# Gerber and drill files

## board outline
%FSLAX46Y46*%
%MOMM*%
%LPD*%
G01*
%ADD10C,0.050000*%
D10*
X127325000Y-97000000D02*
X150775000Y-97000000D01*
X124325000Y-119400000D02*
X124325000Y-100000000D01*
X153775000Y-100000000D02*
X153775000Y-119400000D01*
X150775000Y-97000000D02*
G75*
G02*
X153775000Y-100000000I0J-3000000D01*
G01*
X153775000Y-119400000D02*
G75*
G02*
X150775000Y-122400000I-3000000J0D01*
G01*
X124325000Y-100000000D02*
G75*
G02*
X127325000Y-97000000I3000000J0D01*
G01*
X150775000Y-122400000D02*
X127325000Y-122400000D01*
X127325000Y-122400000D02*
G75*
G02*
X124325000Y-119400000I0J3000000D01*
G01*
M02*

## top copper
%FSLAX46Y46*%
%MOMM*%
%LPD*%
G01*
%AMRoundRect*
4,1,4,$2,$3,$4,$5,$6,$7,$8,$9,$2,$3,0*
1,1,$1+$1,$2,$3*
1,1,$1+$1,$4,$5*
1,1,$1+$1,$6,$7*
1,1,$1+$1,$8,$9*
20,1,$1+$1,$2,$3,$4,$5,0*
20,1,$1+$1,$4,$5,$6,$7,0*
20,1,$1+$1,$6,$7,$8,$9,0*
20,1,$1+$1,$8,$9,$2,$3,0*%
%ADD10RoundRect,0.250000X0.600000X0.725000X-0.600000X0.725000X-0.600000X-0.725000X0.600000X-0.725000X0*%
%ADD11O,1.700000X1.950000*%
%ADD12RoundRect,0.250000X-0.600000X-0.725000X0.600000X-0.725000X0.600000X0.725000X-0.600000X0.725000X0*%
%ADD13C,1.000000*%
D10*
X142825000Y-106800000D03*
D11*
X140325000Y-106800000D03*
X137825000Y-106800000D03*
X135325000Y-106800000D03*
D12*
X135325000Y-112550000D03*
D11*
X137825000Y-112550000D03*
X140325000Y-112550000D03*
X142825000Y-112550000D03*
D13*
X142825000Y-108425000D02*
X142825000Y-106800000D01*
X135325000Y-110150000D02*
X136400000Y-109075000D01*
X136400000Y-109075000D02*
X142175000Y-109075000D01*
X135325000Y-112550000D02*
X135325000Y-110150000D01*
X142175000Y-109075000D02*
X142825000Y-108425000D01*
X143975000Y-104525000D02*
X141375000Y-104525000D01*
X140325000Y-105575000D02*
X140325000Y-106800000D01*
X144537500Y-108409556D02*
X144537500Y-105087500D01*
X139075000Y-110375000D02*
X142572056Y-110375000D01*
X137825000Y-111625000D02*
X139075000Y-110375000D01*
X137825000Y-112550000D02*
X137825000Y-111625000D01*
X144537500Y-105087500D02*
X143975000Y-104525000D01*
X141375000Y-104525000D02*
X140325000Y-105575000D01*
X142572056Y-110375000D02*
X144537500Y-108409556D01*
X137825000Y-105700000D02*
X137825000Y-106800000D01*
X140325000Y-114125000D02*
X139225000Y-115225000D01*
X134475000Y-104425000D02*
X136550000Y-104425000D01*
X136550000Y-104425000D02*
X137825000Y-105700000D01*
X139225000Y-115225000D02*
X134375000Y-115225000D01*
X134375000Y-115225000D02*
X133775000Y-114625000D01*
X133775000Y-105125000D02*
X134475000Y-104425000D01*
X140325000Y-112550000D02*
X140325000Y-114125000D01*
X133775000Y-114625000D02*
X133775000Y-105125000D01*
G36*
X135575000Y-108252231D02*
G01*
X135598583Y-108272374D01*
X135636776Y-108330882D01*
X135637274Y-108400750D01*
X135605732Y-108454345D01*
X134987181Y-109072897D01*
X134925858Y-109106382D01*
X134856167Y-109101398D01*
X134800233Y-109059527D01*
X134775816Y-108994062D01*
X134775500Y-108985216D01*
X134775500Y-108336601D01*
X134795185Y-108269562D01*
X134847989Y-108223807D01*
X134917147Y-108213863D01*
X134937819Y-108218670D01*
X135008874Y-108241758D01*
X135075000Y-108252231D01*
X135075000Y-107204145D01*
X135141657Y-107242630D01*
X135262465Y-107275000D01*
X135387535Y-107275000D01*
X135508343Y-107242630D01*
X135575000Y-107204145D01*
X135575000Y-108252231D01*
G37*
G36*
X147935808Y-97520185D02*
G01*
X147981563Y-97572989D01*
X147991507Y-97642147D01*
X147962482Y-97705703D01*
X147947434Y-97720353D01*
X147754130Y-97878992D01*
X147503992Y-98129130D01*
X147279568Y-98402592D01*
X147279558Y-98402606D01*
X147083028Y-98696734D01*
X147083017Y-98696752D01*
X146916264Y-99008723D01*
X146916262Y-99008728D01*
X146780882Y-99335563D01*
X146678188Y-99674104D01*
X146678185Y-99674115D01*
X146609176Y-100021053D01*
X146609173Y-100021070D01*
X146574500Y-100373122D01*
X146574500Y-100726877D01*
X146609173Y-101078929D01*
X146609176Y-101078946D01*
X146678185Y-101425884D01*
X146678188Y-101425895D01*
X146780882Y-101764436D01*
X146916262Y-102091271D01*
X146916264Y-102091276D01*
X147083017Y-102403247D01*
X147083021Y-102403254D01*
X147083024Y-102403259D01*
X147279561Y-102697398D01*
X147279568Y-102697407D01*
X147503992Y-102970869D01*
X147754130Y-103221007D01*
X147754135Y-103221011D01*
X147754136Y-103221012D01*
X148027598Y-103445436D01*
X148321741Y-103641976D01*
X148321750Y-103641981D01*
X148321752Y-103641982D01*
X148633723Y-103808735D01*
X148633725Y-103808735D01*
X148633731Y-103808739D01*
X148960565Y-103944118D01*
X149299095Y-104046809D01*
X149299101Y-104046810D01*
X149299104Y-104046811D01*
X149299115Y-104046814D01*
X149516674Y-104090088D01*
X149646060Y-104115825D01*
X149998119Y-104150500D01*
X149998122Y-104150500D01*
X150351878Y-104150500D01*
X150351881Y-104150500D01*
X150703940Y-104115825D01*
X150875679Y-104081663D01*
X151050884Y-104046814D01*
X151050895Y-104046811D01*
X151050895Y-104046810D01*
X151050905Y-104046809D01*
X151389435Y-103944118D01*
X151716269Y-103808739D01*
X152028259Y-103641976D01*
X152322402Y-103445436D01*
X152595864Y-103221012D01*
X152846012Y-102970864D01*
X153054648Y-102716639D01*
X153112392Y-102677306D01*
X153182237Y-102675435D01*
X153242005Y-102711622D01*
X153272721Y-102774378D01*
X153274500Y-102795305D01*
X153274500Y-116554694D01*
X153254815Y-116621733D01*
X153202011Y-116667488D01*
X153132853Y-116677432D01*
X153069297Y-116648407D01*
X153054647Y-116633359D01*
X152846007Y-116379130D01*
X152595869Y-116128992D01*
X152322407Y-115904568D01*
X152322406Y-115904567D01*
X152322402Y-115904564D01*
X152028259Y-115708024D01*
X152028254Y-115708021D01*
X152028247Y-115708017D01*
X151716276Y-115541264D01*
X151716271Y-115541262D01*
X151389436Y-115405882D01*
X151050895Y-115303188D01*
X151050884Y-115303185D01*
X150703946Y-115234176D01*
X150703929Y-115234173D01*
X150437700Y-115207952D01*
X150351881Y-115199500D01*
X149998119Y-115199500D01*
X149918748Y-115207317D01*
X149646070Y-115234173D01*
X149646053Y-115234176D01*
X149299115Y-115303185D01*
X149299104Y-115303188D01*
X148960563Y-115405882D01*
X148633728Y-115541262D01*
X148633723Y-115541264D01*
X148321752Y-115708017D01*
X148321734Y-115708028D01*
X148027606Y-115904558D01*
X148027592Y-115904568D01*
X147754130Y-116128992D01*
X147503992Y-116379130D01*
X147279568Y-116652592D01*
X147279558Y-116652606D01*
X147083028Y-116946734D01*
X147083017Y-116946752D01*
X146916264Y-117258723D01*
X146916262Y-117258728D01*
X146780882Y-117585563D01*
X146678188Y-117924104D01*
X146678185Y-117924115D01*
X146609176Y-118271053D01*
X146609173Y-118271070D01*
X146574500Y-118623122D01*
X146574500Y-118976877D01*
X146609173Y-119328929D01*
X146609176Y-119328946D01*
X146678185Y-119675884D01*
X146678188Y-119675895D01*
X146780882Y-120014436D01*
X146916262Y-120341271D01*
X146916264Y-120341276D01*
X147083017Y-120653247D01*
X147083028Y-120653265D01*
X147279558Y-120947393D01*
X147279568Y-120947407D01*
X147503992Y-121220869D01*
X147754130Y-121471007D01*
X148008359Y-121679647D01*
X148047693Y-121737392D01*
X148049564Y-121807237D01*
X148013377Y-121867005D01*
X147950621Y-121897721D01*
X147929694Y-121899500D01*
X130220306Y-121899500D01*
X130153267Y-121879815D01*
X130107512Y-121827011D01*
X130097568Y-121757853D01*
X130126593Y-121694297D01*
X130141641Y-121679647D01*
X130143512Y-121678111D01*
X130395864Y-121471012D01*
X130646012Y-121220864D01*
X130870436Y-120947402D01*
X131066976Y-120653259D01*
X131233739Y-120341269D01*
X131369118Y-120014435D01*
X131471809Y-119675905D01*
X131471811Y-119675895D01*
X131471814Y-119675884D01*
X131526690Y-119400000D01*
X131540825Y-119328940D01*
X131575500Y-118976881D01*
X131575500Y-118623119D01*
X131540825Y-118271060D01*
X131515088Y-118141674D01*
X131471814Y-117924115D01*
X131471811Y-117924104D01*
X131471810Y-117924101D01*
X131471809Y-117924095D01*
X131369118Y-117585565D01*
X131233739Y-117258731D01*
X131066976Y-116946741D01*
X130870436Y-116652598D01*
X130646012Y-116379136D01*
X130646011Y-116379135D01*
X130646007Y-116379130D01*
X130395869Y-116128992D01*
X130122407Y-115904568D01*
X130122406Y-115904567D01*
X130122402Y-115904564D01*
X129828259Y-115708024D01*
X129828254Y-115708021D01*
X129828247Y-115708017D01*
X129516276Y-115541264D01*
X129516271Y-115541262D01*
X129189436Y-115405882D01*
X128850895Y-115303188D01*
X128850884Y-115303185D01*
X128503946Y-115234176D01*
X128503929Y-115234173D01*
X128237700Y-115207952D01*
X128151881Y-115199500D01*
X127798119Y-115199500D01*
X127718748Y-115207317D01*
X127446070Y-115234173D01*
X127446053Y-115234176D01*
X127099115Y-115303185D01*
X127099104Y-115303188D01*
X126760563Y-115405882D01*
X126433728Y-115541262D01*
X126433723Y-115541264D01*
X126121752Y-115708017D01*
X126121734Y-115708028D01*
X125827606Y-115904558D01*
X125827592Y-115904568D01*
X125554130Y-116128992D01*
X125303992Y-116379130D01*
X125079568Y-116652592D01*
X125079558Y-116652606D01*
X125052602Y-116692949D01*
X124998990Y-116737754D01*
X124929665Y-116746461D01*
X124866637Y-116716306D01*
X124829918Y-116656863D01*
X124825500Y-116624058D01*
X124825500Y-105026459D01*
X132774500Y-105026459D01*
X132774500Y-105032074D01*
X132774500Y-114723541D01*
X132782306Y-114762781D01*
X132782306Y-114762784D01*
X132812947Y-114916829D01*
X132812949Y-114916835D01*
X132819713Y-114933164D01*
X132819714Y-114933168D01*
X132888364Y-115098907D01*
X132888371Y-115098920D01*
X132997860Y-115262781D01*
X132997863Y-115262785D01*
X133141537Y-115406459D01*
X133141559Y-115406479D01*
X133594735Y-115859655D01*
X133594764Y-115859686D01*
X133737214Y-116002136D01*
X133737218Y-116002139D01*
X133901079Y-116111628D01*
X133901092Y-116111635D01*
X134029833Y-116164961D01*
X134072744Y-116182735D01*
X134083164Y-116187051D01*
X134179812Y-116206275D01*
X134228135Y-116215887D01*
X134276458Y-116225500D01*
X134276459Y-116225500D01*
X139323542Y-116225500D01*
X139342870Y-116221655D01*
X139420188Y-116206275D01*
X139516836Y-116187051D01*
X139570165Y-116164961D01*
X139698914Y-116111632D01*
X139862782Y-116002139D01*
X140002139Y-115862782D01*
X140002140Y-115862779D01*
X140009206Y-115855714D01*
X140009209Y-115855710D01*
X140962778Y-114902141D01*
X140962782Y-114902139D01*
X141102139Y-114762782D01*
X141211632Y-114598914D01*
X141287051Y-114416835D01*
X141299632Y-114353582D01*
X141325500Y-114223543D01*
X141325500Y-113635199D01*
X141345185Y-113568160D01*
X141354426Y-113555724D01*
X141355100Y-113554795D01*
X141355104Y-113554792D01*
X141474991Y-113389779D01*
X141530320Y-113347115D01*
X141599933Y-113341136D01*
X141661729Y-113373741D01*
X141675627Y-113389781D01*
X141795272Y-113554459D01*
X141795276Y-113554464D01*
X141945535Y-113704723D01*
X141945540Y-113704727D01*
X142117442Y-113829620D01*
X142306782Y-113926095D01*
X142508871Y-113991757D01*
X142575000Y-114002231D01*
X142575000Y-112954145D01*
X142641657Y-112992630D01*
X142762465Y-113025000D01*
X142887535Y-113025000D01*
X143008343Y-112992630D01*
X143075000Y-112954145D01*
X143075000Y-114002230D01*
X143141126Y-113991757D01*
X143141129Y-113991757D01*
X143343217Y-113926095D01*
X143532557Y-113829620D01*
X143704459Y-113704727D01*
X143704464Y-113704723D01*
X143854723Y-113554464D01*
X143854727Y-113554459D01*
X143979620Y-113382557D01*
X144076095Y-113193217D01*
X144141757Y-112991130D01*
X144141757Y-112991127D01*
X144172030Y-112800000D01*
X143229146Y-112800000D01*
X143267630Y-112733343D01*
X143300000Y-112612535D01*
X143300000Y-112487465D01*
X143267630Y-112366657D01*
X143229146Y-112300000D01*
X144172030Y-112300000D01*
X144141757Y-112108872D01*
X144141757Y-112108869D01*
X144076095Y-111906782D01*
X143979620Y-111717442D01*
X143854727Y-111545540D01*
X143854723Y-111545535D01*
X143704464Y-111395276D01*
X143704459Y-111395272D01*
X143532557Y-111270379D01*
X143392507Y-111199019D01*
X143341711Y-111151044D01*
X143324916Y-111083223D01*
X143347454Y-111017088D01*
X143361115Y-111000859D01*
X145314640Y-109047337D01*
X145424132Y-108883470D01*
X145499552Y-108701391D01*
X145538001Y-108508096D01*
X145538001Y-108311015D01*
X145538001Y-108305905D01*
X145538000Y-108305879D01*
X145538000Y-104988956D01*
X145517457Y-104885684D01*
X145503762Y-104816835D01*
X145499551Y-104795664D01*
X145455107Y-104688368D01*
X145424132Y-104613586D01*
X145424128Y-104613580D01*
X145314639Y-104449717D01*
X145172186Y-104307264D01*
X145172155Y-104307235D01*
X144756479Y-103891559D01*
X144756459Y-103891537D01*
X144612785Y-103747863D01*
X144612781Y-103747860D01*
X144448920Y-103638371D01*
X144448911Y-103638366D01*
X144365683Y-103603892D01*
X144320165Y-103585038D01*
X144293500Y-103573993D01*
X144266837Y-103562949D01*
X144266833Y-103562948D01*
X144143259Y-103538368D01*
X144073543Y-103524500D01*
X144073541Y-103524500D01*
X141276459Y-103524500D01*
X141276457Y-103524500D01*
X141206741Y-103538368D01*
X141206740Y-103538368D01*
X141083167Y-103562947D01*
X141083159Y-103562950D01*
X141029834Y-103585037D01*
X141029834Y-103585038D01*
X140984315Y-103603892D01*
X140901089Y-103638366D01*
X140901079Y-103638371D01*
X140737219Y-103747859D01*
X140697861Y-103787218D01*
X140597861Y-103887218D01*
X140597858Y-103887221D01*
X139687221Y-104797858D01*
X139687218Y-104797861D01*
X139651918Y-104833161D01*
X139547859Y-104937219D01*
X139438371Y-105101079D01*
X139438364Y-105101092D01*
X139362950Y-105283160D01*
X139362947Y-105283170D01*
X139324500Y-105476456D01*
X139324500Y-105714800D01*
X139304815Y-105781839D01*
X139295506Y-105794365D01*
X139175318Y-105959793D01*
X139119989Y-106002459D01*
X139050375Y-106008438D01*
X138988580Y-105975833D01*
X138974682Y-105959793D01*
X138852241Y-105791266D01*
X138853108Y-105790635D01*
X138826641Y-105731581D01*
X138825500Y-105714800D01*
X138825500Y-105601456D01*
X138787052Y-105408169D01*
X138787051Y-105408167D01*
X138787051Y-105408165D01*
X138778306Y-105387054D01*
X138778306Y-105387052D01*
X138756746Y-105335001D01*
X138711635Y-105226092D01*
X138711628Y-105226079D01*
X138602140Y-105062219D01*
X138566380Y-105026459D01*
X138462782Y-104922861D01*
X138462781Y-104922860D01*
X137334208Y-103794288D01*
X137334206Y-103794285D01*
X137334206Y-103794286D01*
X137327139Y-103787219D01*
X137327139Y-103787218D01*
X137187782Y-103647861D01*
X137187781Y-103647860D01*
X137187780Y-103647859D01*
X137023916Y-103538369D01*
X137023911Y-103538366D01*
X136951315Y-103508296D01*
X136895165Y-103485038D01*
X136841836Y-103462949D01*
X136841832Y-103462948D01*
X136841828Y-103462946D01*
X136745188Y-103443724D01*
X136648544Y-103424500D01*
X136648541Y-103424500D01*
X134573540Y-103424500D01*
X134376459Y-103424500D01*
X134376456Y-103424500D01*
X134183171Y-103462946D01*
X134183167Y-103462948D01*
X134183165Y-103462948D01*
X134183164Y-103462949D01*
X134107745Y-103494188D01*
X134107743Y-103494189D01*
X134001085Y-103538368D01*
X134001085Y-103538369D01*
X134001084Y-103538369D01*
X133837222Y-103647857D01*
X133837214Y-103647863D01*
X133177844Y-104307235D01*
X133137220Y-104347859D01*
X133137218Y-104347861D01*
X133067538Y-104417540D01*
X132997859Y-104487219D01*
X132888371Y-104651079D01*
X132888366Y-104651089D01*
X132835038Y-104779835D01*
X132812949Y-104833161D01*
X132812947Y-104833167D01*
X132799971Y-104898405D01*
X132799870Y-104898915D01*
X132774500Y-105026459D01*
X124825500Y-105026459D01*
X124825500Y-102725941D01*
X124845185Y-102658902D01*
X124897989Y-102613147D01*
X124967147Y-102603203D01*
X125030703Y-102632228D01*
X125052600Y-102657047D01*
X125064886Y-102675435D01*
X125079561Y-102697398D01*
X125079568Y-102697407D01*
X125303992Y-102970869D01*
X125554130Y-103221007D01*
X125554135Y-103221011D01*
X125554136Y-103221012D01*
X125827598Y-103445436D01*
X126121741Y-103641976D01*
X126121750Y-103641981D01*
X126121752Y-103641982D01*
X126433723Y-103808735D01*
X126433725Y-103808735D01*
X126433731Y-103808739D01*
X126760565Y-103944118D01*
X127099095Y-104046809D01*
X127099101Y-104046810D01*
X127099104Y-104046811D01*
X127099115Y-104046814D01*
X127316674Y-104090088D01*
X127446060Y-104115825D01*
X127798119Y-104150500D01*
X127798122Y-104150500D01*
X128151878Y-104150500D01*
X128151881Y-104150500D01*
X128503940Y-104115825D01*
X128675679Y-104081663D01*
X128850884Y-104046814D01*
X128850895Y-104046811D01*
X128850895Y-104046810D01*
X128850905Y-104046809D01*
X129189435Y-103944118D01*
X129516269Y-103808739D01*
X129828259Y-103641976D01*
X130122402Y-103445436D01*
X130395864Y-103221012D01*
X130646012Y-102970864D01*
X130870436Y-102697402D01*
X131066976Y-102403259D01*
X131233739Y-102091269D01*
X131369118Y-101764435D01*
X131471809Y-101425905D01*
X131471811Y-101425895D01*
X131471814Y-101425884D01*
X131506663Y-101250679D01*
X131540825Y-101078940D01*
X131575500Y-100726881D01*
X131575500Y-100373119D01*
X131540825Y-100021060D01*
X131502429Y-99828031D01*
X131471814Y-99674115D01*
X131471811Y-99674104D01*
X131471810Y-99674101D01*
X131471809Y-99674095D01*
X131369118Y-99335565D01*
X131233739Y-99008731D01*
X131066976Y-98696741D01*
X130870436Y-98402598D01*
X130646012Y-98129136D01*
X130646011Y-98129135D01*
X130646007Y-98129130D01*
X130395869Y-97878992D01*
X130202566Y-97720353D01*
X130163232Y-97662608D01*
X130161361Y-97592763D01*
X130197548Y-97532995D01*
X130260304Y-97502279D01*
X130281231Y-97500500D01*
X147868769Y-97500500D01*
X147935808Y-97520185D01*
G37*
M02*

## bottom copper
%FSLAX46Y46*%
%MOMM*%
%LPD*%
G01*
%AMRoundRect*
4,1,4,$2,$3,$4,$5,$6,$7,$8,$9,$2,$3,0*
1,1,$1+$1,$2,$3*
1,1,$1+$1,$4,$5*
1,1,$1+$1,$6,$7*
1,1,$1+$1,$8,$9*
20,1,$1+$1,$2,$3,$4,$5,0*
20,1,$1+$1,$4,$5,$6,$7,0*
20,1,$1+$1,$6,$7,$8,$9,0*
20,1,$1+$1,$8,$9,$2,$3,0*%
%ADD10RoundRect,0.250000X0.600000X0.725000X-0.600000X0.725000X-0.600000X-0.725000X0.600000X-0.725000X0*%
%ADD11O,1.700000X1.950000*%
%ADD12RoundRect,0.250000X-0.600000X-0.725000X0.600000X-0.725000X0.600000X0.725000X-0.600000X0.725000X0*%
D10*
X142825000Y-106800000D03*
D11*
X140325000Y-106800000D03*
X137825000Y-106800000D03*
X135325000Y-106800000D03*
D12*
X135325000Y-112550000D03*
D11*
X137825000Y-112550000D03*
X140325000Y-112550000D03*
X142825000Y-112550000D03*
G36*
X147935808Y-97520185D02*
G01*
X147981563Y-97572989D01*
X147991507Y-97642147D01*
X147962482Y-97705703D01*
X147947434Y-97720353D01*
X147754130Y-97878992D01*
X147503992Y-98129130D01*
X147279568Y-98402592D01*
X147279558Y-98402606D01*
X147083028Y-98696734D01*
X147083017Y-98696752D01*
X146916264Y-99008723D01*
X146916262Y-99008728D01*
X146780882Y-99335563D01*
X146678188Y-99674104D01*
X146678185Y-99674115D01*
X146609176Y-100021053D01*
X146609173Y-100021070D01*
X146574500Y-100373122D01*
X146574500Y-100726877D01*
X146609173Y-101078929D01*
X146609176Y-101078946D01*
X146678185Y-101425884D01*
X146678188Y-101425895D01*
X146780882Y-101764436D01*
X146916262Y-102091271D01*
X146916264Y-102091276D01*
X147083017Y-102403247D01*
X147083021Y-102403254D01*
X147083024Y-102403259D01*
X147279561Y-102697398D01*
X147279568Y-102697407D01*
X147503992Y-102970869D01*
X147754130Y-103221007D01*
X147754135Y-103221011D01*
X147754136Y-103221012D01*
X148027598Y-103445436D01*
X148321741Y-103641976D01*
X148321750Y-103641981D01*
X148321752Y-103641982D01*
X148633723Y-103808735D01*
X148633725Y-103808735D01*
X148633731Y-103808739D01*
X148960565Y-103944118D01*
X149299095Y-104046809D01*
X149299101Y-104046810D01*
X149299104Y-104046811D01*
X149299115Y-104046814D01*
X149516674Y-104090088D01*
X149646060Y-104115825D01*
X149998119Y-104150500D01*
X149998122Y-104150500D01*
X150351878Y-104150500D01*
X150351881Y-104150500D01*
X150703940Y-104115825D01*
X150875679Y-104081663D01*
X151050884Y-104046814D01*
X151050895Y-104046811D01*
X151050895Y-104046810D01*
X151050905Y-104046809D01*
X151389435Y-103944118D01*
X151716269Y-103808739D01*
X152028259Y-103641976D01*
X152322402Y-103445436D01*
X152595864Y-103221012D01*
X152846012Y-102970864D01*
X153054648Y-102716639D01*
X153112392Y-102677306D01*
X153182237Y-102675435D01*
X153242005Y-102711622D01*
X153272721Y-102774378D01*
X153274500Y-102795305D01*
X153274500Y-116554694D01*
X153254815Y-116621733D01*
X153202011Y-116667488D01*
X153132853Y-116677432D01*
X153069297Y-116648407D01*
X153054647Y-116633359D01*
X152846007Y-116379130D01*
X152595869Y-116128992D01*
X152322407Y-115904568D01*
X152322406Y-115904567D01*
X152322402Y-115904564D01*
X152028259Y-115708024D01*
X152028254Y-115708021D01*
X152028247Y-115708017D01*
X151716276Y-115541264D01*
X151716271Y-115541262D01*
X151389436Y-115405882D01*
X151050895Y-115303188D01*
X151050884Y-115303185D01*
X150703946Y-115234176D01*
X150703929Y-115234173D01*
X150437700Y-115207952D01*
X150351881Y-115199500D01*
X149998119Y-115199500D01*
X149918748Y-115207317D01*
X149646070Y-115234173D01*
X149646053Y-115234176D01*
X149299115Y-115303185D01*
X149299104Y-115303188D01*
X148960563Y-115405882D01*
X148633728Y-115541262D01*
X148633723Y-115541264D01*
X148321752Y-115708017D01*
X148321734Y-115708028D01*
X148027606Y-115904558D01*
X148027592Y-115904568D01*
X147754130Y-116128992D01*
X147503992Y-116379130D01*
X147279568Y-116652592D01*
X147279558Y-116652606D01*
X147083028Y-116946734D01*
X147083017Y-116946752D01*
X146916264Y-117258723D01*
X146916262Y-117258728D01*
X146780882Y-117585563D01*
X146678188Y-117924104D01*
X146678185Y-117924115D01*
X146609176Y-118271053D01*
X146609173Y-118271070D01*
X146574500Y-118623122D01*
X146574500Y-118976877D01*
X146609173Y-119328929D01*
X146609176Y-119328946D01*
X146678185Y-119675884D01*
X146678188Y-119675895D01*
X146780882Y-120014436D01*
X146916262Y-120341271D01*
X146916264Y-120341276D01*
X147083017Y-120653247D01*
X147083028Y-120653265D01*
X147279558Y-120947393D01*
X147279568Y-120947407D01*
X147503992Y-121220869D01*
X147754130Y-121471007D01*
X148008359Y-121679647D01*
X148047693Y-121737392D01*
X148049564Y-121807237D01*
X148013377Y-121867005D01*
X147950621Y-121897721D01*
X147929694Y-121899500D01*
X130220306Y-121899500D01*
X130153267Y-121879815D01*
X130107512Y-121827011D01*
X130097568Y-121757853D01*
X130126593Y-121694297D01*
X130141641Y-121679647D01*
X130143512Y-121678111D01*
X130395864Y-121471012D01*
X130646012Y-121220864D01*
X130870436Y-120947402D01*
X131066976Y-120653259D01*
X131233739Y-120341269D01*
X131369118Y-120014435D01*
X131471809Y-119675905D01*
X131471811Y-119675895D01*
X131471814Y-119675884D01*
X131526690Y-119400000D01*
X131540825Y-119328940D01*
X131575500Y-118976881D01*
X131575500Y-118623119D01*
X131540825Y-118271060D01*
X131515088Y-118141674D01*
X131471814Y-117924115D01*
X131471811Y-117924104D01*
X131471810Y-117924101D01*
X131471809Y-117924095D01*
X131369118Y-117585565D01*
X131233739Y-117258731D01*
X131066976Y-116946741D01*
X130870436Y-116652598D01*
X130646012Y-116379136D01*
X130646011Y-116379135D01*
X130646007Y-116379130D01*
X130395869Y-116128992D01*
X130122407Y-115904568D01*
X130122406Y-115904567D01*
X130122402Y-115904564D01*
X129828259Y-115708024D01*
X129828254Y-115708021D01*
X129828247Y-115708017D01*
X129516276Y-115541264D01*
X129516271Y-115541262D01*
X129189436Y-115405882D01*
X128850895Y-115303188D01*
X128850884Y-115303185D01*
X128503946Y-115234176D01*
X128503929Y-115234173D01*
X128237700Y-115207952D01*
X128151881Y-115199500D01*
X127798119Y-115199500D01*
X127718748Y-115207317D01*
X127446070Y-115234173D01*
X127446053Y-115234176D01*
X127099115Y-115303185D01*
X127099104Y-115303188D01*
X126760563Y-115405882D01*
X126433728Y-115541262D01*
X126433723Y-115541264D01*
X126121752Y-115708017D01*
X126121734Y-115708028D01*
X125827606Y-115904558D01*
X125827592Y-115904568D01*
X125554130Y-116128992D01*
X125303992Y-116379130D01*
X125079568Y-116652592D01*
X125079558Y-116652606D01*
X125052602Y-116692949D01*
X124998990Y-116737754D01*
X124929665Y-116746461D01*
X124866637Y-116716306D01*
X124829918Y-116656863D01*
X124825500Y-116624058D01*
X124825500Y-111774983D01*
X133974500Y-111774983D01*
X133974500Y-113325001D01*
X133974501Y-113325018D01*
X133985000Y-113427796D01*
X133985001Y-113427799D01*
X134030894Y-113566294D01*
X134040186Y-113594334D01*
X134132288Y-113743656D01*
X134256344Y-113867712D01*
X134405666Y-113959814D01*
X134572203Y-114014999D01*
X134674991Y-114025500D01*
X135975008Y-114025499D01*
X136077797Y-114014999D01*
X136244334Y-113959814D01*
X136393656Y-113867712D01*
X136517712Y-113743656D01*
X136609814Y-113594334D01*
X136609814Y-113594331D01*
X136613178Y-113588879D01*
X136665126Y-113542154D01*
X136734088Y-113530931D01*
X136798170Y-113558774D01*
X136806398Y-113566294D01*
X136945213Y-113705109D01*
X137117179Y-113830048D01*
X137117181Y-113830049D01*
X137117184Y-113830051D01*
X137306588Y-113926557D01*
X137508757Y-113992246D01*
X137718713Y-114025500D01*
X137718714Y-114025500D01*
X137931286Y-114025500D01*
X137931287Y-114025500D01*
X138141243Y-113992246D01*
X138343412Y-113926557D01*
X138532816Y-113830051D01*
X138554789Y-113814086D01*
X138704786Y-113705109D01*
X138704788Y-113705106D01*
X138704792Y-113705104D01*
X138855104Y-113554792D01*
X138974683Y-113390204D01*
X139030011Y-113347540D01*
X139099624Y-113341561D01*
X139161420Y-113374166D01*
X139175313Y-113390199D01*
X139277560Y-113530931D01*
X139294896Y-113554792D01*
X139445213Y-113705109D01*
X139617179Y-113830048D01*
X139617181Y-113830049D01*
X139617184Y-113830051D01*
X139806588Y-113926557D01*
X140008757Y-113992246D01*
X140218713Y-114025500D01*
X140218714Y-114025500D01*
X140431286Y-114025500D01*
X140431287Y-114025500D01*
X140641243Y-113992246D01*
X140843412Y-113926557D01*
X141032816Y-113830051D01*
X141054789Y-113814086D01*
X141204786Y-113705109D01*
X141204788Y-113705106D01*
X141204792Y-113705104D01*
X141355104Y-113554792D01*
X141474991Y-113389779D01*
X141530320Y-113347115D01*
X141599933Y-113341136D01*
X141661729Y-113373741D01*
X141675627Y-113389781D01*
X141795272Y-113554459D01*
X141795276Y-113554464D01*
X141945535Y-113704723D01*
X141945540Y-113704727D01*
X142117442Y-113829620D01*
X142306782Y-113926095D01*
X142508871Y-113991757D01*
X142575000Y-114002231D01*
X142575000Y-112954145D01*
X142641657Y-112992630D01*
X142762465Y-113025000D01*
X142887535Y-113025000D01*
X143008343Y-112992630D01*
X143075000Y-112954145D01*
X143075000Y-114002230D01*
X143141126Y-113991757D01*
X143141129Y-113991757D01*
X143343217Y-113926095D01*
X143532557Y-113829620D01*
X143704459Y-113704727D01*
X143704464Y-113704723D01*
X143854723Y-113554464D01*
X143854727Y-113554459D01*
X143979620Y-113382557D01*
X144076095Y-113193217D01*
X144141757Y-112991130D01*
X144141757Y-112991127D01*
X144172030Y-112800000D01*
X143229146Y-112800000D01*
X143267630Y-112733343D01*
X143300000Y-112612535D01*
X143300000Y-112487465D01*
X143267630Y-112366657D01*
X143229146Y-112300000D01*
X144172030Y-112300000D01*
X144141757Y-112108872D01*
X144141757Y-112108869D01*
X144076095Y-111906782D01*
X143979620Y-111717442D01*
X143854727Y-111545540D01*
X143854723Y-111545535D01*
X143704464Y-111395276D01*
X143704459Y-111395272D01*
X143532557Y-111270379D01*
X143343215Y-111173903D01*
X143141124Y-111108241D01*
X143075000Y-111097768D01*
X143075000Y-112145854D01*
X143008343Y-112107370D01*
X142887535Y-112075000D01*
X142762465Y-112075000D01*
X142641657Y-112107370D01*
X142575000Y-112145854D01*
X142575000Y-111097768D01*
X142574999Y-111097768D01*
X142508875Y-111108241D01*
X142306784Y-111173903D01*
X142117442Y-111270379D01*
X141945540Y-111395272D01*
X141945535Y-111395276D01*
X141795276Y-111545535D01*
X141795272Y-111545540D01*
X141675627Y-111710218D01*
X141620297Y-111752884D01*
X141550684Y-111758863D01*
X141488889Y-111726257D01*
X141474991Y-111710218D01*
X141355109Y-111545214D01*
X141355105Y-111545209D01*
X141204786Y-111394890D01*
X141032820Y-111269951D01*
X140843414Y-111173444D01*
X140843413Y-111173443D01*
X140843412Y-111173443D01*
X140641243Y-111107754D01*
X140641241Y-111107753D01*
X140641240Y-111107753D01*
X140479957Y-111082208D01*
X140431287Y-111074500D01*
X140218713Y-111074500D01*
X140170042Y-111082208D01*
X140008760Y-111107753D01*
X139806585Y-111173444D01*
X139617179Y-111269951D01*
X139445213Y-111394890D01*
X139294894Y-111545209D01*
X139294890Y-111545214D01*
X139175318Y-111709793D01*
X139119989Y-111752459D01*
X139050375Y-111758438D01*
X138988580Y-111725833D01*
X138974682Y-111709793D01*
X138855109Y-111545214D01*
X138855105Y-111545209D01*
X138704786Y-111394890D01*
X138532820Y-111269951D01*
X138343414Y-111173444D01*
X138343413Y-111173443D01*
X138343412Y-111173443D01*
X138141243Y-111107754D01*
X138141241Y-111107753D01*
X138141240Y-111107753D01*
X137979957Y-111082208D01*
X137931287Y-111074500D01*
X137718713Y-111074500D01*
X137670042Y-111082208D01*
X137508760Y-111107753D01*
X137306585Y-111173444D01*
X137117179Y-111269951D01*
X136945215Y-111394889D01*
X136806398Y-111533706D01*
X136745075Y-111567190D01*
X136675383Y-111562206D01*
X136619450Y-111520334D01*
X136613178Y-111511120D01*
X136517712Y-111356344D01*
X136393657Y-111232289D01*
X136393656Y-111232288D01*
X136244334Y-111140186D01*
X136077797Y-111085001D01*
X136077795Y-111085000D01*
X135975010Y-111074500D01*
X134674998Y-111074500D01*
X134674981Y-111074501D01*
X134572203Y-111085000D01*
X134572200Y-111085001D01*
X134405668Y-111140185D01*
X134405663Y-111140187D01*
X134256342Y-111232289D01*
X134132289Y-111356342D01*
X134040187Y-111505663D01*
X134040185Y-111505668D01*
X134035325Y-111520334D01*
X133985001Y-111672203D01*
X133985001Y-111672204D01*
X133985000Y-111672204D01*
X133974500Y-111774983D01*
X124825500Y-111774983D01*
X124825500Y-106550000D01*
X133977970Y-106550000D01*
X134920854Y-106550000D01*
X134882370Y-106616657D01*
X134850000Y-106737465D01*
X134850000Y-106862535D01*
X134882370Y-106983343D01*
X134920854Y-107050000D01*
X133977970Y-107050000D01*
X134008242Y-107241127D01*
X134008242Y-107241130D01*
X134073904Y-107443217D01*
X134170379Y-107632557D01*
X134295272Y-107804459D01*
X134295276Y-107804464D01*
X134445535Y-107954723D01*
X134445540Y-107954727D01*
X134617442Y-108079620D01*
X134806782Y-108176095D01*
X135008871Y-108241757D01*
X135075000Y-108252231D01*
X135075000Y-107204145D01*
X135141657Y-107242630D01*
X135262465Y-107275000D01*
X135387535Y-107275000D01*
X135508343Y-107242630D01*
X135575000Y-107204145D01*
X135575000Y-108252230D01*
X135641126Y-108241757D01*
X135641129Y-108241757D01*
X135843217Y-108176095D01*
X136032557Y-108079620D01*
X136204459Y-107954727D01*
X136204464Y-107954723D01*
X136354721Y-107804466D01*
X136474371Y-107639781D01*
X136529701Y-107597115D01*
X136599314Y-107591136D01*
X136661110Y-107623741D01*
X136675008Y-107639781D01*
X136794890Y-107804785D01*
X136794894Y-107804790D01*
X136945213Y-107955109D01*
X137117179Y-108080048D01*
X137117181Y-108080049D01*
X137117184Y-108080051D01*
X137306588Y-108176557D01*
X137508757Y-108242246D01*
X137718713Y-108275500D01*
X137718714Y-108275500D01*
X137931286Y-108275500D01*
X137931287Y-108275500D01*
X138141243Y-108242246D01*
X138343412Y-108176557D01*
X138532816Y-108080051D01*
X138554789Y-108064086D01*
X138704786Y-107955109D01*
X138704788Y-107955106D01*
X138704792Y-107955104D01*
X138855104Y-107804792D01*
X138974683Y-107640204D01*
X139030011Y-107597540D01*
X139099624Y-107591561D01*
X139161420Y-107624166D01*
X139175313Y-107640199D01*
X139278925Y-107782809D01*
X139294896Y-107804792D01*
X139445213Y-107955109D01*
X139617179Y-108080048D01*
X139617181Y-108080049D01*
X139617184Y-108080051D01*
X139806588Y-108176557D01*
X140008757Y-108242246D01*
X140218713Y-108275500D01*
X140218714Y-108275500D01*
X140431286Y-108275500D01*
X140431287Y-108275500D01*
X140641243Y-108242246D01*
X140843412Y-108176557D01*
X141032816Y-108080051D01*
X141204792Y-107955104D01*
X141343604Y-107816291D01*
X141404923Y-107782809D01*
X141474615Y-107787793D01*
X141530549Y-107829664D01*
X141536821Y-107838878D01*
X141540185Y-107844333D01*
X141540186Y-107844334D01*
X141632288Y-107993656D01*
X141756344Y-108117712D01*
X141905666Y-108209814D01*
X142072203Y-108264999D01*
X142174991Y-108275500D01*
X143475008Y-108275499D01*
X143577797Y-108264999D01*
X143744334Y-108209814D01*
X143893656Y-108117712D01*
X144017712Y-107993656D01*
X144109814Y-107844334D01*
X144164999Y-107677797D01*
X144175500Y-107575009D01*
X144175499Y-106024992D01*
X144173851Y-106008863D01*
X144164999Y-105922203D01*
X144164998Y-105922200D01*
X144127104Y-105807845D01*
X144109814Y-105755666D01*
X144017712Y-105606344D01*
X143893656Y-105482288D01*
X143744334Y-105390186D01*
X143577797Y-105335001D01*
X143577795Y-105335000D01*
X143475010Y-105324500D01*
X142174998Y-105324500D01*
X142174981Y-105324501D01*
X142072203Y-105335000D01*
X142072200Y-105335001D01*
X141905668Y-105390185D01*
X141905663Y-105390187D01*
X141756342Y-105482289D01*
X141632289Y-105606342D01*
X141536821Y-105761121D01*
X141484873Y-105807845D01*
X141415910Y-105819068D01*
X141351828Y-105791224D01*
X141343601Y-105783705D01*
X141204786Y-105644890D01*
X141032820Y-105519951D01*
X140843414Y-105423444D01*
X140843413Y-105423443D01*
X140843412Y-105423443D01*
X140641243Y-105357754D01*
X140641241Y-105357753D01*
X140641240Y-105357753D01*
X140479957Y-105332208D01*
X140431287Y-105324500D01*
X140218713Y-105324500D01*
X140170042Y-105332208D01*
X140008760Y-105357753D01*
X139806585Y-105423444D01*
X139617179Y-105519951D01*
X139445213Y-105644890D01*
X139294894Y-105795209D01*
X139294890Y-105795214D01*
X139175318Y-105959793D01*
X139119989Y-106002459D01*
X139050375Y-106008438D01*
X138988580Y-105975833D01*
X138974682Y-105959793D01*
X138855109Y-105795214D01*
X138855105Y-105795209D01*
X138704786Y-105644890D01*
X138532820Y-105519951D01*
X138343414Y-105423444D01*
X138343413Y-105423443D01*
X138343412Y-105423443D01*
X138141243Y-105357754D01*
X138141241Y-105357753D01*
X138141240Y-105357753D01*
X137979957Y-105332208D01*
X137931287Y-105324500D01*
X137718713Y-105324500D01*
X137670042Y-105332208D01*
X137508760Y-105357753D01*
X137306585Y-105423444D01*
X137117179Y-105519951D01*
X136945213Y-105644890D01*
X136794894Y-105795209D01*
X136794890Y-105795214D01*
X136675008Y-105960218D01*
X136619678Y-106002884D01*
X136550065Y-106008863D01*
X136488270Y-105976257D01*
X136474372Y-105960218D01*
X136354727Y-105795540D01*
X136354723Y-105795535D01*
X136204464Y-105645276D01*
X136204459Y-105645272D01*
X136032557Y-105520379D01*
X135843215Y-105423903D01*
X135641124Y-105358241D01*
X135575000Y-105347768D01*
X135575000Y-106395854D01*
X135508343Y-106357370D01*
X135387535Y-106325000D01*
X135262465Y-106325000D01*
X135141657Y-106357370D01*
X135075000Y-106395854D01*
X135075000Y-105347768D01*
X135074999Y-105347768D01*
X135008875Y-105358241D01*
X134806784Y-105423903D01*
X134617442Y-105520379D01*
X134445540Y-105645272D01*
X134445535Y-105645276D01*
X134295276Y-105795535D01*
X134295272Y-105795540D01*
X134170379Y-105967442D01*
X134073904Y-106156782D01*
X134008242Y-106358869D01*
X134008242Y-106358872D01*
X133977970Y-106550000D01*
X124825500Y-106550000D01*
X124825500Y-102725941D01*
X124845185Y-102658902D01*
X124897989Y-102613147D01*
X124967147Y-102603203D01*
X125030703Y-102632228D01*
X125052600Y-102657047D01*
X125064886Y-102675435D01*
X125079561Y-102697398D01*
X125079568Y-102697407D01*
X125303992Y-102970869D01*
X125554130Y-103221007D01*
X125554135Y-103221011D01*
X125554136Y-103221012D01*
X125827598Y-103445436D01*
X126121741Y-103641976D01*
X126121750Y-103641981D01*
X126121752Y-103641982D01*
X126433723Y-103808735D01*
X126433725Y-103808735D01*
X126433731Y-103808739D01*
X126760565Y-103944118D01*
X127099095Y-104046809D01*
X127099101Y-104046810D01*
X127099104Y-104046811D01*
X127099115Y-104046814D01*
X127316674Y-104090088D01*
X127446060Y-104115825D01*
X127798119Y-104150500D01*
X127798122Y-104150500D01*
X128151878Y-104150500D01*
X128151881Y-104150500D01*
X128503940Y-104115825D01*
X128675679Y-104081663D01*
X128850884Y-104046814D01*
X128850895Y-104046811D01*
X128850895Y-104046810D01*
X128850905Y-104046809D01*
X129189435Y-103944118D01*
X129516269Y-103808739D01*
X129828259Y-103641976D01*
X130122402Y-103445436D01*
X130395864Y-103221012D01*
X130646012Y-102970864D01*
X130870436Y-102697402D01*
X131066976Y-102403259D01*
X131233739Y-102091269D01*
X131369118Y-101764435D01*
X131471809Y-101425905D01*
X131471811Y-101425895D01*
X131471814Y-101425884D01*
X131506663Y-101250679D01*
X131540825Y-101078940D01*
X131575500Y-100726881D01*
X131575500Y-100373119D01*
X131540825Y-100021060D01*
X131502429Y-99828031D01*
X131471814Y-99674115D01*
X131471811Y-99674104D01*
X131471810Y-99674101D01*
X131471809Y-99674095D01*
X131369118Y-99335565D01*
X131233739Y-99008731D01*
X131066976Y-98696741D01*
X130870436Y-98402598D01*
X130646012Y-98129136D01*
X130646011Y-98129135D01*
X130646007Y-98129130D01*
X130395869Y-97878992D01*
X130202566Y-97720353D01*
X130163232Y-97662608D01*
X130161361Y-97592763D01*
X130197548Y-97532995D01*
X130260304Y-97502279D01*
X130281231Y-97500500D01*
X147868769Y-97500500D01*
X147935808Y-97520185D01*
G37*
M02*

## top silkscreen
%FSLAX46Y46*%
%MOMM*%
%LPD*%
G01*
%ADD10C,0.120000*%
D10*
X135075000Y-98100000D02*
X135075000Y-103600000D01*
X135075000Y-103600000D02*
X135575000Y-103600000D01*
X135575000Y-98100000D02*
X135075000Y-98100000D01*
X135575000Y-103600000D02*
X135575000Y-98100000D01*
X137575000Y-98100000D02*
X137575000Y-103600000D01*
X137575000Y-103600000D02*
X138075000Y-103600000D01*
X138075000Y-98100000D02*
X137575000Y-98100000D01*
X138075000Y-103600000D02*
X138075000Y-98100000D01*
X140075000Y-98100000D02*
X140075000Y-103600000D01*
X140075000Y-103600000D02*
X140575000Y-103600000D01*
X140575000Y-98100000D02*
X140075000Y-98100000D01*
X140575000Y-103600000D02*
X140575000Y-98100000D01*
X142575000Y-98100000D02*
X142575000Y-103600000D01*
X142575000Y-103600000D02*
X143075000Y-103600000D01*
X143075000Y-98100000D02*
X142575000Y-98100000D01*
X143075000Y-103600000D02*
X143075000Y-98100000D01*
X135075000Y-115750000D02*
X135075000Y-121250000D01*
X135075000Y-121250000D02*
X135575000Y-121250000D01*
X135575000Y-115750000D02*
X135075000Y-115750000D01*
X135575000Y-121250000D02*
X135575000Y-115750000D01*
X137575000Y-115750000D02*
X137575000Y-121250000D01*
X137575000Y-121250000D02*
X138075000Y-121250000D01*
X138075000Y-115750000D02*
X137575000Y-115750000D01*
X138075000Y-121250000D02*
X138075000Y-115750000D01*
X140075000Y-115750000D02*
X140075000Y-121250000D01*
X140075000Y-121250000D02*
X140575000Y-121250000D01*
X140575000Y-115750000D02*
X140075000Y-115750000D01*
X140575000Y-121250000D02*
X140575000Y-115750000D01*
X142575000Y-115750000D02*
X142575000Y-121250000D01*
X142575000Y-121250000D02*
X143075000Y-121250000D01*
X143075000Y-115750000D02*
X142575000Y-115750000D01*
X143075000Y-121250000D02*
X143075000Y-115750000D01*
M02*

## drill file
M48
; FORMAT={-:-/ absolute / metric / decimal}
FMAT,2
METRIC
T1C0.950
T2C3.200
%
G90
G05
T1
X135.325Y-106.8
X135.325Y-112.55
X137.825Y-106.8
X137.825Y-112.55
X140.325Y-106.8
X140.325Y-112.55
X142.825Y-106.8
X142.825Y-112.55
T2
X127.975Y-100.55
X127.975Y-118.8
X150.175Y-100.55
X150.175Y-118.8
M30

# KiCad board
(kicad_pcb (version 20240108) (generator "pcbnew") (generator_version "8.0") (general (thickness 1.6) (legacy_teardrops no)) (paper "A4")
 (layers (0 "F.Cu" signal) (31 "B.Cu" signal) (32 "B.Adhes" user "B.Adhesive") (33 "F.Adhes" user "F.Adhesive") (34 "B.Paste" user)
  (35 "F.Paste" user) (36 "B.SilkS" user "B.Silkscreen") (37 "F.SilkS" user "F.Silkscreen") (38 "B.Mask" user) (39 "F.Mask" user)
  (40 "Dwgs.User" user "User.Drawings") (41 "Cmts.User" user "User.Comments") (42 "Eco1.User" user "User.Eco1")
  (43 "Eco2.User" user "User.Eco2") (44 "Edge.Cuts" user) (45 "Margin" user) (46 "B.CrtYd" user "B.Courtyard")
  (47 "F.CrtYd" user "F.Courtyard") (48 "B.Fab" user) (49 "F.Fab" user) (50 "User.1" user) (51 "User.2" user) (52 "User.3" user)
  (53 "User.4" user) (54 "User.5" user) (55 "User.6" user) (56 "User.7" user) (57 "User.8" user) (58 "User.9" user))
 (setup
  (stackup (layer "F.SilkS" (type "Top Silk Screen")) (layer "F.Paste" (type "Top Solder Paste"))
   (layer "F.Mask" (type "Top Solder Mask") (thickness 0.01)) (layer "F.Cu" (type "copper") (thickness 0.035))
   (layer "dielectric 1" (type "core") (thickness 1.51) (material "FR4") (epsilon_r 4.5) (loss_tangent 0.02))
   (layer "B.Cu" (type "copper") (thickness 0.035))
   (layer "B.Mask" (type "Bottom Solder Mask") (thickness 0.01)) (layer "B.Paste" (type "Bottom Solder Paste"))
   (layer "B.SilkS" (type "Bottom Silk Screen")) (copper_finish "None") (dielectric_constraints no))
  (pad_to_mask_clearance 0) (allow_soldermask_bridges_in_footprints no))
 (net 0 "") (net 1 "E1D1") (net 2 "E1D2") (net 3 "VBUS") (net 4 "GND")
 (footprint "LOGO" (layer "F.Cu") (at 146.350293 109.852368)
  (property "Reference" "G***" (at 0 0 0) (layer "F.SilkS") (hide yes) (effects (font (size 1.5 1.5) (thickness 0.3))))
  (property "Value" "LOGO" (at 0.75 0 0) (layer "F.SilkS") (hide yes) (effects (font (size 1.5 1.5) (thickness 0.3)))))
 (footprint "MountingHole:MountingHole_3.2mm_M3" (layer "F.Cu") (at 150.175 118.8)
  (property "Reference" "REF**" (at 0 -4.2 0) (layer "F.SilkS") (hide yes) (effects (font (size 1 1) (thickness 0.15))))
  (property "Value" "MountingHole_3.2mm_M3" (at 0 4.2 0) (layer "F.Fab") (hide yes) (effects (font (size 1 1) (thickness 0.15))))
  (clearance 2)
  (pad "" np_thru_hole circle (at 0 0) (size 3.2 3.2) (drill 3.2) (layers "*.Cu" "*.Mask")))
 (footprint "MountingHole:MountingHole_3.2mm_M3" (layer "F.Cu") (at 150.175 100.55)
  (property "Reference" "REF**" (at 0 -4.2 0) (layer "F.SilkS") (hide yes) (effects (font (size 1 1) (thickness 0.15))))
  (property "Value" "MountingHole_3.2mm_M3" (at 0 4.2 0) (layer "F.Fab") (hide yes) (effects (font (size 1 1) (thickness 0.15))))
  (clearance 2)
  (pad "" np_thru_hole circle (at 0 0) (size 3.2 3.2) (drill 3.2) (layers "*.Cu" "*.Mask")))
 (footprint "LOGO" (layer "F.Cu") (at 132.30565 109.62003)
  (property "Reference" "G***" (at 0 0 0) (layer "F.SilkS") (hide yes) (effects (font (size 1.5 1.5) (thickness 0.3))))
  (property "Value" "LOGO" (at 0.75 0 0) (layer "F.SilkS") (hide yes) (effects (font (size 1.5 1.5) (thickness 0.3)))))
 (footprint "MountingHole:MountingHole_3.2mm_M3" (layer "F.Cu") (at 127.975 118.8)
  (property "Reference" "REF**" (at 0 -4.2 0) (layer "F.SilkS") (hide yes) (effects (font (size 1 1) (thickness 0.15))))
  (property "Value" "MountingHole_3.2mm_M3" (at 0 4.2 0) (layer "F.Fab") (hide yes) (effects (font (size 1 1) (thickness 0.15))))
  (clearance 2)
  (pad "" np_thru_hole circle (at 0 0) (size 3.2 3.2) (drill 3.2) (layers "*.Cu" "*.Mask")))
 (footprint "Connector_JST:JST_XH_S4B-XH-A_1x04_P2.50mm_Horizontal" (layer "F.Cu") (at 142.825 106.8 180)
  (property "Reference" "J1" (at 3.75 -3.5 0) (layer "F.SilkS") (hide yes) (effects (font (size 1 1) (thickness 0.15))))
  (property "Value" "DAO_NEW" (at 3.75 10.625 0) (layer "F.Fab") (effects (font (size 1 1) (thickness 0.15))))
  (fp_line (start 7.75 8.7) (end 7.75 3.2) (stroke (width 0.12) (type solid)) (layer "F.SilkS"))
  (fp_line (start 7.75 3.2) (end 7.25 3.2) (stroke (width 0.12) (type solid)) (layer "F.SilkS"))
  (fp_line (start 7.25 8.7) (end 7.75 8.7) (stroke (width 0.12) (type solid)) (layer "F.SilkS"))
  (fp_line (start 7.25 3.2) (end 7.25 8.7) (stroke (width 0.12) (type solid)) (layer "F.SilkS"))
  (fp_line (start 5.25 8.7) (end 5.25 3.2) (stroke (width 0.12) (type solid)) (layer "F.SilkS"))
  (fp_line (start 5.25 3.2) (end 4.75 3.2) (stroke (width 0.12) (type solid)) (layer "F.SilkS"))
  (fp_line (start 4.75 8.7) (end 5.25 8.7) (stroke (width 0.12) (type solid)) (layer "F.SilkS"))
  (fp_line (start 4.75 3.2) (end 4.75 8.7) (stroke (width 0.12) (type solid)) (layer "F.SilkS"))
  (fp_line (start 2.75 8.7) (end 2.75 3.2) (stroke (width 0.12) (type solid)) (layer "F.SilkS"))
  (fp_line (start 2.75 3.2) (end 2.25 3.2) (stroke (width 0.12) (type solid)) (layer "F.SilkS"))
  (fp_line (start 2.25 8.7) (end 2.75 8.7) (stroke (width 0.12) (type solid)) (layer "F.SilkS"))
  (fp_line (start 2.25 3.2) (end 2.25 8.7) (stroke (width 0.12) (type solid)) (layer "F.SilkS"))
  (fp_line (start 0.25 8.7) (end 0.25 3.2) (stroke (width 0.12) (type solid)) (layer "F.SilkS"))
  (fp_line (start 0.25 3.2) (end -0.25 3.2) (stroke (width 0.12) (type solid)) (layer "F.SilkS"))
  (fp_line (start -0.25 8.7) (end 0.25 8.7) (stroke (width 0.12) (type solid)) (layer "F.SilkS"))
  (fp_line (start -0.25 3.2) (end -0.25 8.7) (stroke (width 0.12) (type solid)) (layer "F.SilkS"))
  (pad "1" thru_hole roundrect (at 0 0 180) (size 1.7 1.95) (drill 0.95) (layers "*.Cu" "*.Mask") (remove_unused_layers no)
   (roundrect_rratio 0.147059) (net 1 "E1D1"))
  (pad "2" thru_hole oval (at 2.5 0 180) (size 1.7 1.95) (drill 0.95) (layers "*.Cu" "*.Mask") (remove_unused_layers no) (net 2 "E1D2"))
  (pad "3" thru_hole oval (at 5 0 180) (size 1.7 1.95) (drill 0.95) (layers "*.Cu" "*.Mask") (remove_unused_layers no) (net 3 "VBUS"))
  (pad "4" thru_hole oval (at 7.5 0 180) (size 1.7 1.95) (drill 0.95) (layers "*.Cu" "*.Mask") (remove_unused_layers no) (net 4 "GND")))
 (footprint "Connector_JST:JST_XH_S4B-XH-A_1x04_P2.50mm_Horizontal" (layer "F.Cu") (at 135.325 112.55)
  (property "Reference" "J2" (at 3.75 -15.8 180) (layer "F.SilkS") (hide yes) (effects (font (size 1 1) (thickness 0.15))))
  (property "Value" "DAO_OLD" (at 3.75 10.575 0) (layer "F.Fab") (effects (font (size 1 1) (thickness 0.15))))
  (fp_line (start -0.25 3.2) (end -0.25 8.7) (stroke (width 0.12) (type solid)) (layer "F.SilkS"))
  (fp_line (start -0.25 8.7) (end 0.25 8.7) (stroke (width 0.12) (type solid)) (layer "F.SilkS"))
  (fp_line (start 0.25 3.2) (end -0.25 3.2) (stroke (width 0.12) (type solid)) (layer "F.SilkS"))
  (fp_line (start 0.25 8.7) (end 0.25 3.2) (stroke (width 0.12) (type solid)) (layer "F.SilkS"))
  (fp_line (start 2.25 3.2) (end 2.25 8.7) (stroke (width 0.12) (type solid)) (layer "F.SilkS"))
  (fp_line (start 2.25 8.7) (end 2.75 8.7) (stroke (width 0.12) (type solid)) (layer "F.SilkS"))
  (fp_line (start 2.75 3.2) (end 2.25 3.2) (stroke (width 0.12) (type solid)) (layer "F.SilkS"))
  (fp_line (start 2.75 8.7) (end 2.75 3.2) (stroke (width 0.12) (type solid)) (layer "F.SilkS"))
  (fp_line (start 4.75 3.2) (end 4.75 8.7) (stroke (width 0.12) (type solid)) (layer "F.SilkS"))
  (fp_line (start 4.75 8.7) (end 5.25 8.7) (stroke (width 0.12) (type solid)) (layer "F.SilkS"))
  (fp_line (start 5.25 3.2) (end 4.75 3.2) (stroke (width 0.12) (type solid)) (layer "F.SilkS"))
  (fp_line (start 5.25 8.7) (end 5.25 3.2) (stroke (width 0.12) (type solid)) (layer "F.SilkS"))
  (fp_line (start 7.25 3.2) (end 7.25 8.7) (stroke (width 0.12) (type solid)) (layer "F.SilkS"))
  (fp_line (start 7.25 8.7) (end 7.75 8.7) (stroke (width 0.12) (type solid)) (layer "F.SilkS"))
  (fp_line (start 7.75 3.2) (end 7.25 3.2) (stroke (width 0.12) (type solid)) (layer "F.SilkS"))
  (fp_line (start 7.75 8.7) (end 7.75 3.2) (stroke (width 0.12) (type solid)) (layer "F.SilkS"))
  (pad "1" thru_hole roundrect (at 0 0) (size 1.7 1.95) (drill 0.95) (layers "*.Cu" "*.Mask") (remove_unused_layers no)
   (roundrect_rratio 0.147059) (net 1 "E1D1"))
  (pad "2" thru_hole oval (at 2.5 0) (size 1.7 1.95) (drill 0.95) (layers "*.Cu" "*.Mask") (remove_unused_layers no) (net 2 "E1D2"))
  (pad "3" thru_hole oval (at 5 0) (size 1.7 1.95) (drill 0.95) (layers "*.Cu" "*.Mask") (remove_unused_layers no) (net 3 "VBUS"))
  (pad "4" thru_hole oval (at 7.5 0) (size 1.7 1.95) (drill 0.95) (layers "*.Cu" "*.Mask") (remove_unused_layers no) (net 4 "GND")))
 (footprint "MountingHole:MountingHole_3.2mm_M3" (layer "F.Cu") (at 127.975 100.55)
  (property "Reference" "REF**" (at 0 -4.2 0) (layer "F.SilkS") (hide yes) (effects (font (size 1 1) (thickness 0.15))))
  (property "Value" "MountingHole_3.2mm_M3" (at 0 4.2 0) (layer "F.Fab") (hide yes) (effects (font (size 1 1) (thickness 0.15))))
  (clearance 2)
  (pad "" np_thru_hole circle (at 0 0) (size 3.2 3.2) (drill 3.2) (layers "*.Cu" "*.Mask")))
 (gr_line (start 127.325 97) (end 150.775 97) (stroke (width 0.05) (type default)) (layer "Edge.Cuts"))
 (gr_line (start 124.325 119.4) (end 124.325 100) (stroke (width 0.05) (type default)) (layer "Edge.Cuts"))
 (gr_line (start 153.775 100) (end 153.775 119.4) (stroke (width 0.05) (type default)) (layer "Edge.Cuts"))
 (gr_arc (start 150.775 97) (mid 152.89632 97.87868) (end 153.775 100) (stroke (width 0.05) (type default)) (layer "Edge.Cuts"))
 (gr_arc (start 153.775 119.4) (mid 152.89632 121.52132) (end 150.775 122.4) (stroke (width 0.05) (type default)) (layer "Edge.Cuts"))
 (gr_arc (start 124.325 100) (mid 125.20368 97.87868) (end 127.325 97) (stroke (width 0.05) (type default)) (layer "Edge.Cuts"))
 (gr_line (start 150.775 122.4) (end 127.325 122.4) (stroke (width 0.05) (type default)) (layer "Edge.Cuts"))
 (gr_arc (start 127.325 122.4) (mid 125.20368 121.52132) (end 124.325 119.4) (stroke (width 0.05) (type default)) (layer "Edge.Cuts"))
 (segment (start 142.825 108.425) (end 142.825 106.8) (width 1) (layer "F.Cu") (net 1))
 (segment (start 135.325 110.15) (end 136.4 109.075) (width 1) (layer "F.Cu") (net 1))
 (segment (start 136.4 109.075) (end 142.175 109.075) (width 1) (layer "F.Cu") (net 1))
 (segment (start 135.325 112.55) (end 135.325 110.15) (width 1) (layer "F.Cu") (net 1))
 (segment (start 142.175 109.075) (end 142.825 108.425) (width 1) (layer "F.Cu") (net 1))
 (segment (start 143.975 104.525) (end 141.375 104.525) (width 1) (layer "F.Cu") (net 2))
 (segment (start 140.325 105.575) (end 140.325 106.8) (width 1) (layer "F.Cu") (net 2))
 (segment (start 144.5375 108.409556) (end 144.5375 105.0875) (width 1) (layer "F.Cu") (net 2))
 (segment (start 139.075 110.375) (end 142.572056 110.375) (width 1) (layer "F.Cu") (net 2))
 (segment (start 137.825 111.625) (end 139.075 110.375) (width 1) (layer "F.Cu") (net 2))
 (segment (start 137.825 112.55) (end 137.825 111.625) (width 1) (layer "F.Cu") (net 2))
 (segment (start 144.5375 105.0875) (end 143.975 104.525) (width 1) (layer "F.Cu") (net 2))
 (segment (start 141.375 104.525) (end 140.325 105.575) (width 1) (layer "F.Cu") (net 2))
 (segment (start 142.572056 110.375) (end 144.5375 108.409556) (width 1) (layer "F.Cu") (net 2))
 (segment (start 137.825 105.7) (end 137.825 106.8) (width 1) (layer "F.Cu") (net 3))
 (segment (start 140.325 114.125) (end 139.225 115.225) (width 1) (layer "F.Cu") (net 3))
 (segment (start 134.475 104.425) (end 136.55 104.425) (width 1) (layer "F.Cu") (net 3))
 (segment (start 136.55 104.425) (end 137.825 105.7) (width 1) (layer "F.Cu") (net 3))
 (segment (start 139.225 115.225) (end 134.375 115.225) (width 1) (layer "F.Cu") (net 3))
 (segment (start 134.375 115.225) (end 133.775 114.625) (width 1) (layer "F.Cu") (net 3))
 (segment (start 133.775 105.125) (end 134.475 104.425) (width 1) (layer "F.Cu") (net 3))
 (segment (start 140.325 112.55) (end 140.325 114.125) (width 1) (layer "F.Cu") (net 3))
 (segment (start 133.775 114.625) (end 133.775 105.125) (width 1) (layer "F.Cu") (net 3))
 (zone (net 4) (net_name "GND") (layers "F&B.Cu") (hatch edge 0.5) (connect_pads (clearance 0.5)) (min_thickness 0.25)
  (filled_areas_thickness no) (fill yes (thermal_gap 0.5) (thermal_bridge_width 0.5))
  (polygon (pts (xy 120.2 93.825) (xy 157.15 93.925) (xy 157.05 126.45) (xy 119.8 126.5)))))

